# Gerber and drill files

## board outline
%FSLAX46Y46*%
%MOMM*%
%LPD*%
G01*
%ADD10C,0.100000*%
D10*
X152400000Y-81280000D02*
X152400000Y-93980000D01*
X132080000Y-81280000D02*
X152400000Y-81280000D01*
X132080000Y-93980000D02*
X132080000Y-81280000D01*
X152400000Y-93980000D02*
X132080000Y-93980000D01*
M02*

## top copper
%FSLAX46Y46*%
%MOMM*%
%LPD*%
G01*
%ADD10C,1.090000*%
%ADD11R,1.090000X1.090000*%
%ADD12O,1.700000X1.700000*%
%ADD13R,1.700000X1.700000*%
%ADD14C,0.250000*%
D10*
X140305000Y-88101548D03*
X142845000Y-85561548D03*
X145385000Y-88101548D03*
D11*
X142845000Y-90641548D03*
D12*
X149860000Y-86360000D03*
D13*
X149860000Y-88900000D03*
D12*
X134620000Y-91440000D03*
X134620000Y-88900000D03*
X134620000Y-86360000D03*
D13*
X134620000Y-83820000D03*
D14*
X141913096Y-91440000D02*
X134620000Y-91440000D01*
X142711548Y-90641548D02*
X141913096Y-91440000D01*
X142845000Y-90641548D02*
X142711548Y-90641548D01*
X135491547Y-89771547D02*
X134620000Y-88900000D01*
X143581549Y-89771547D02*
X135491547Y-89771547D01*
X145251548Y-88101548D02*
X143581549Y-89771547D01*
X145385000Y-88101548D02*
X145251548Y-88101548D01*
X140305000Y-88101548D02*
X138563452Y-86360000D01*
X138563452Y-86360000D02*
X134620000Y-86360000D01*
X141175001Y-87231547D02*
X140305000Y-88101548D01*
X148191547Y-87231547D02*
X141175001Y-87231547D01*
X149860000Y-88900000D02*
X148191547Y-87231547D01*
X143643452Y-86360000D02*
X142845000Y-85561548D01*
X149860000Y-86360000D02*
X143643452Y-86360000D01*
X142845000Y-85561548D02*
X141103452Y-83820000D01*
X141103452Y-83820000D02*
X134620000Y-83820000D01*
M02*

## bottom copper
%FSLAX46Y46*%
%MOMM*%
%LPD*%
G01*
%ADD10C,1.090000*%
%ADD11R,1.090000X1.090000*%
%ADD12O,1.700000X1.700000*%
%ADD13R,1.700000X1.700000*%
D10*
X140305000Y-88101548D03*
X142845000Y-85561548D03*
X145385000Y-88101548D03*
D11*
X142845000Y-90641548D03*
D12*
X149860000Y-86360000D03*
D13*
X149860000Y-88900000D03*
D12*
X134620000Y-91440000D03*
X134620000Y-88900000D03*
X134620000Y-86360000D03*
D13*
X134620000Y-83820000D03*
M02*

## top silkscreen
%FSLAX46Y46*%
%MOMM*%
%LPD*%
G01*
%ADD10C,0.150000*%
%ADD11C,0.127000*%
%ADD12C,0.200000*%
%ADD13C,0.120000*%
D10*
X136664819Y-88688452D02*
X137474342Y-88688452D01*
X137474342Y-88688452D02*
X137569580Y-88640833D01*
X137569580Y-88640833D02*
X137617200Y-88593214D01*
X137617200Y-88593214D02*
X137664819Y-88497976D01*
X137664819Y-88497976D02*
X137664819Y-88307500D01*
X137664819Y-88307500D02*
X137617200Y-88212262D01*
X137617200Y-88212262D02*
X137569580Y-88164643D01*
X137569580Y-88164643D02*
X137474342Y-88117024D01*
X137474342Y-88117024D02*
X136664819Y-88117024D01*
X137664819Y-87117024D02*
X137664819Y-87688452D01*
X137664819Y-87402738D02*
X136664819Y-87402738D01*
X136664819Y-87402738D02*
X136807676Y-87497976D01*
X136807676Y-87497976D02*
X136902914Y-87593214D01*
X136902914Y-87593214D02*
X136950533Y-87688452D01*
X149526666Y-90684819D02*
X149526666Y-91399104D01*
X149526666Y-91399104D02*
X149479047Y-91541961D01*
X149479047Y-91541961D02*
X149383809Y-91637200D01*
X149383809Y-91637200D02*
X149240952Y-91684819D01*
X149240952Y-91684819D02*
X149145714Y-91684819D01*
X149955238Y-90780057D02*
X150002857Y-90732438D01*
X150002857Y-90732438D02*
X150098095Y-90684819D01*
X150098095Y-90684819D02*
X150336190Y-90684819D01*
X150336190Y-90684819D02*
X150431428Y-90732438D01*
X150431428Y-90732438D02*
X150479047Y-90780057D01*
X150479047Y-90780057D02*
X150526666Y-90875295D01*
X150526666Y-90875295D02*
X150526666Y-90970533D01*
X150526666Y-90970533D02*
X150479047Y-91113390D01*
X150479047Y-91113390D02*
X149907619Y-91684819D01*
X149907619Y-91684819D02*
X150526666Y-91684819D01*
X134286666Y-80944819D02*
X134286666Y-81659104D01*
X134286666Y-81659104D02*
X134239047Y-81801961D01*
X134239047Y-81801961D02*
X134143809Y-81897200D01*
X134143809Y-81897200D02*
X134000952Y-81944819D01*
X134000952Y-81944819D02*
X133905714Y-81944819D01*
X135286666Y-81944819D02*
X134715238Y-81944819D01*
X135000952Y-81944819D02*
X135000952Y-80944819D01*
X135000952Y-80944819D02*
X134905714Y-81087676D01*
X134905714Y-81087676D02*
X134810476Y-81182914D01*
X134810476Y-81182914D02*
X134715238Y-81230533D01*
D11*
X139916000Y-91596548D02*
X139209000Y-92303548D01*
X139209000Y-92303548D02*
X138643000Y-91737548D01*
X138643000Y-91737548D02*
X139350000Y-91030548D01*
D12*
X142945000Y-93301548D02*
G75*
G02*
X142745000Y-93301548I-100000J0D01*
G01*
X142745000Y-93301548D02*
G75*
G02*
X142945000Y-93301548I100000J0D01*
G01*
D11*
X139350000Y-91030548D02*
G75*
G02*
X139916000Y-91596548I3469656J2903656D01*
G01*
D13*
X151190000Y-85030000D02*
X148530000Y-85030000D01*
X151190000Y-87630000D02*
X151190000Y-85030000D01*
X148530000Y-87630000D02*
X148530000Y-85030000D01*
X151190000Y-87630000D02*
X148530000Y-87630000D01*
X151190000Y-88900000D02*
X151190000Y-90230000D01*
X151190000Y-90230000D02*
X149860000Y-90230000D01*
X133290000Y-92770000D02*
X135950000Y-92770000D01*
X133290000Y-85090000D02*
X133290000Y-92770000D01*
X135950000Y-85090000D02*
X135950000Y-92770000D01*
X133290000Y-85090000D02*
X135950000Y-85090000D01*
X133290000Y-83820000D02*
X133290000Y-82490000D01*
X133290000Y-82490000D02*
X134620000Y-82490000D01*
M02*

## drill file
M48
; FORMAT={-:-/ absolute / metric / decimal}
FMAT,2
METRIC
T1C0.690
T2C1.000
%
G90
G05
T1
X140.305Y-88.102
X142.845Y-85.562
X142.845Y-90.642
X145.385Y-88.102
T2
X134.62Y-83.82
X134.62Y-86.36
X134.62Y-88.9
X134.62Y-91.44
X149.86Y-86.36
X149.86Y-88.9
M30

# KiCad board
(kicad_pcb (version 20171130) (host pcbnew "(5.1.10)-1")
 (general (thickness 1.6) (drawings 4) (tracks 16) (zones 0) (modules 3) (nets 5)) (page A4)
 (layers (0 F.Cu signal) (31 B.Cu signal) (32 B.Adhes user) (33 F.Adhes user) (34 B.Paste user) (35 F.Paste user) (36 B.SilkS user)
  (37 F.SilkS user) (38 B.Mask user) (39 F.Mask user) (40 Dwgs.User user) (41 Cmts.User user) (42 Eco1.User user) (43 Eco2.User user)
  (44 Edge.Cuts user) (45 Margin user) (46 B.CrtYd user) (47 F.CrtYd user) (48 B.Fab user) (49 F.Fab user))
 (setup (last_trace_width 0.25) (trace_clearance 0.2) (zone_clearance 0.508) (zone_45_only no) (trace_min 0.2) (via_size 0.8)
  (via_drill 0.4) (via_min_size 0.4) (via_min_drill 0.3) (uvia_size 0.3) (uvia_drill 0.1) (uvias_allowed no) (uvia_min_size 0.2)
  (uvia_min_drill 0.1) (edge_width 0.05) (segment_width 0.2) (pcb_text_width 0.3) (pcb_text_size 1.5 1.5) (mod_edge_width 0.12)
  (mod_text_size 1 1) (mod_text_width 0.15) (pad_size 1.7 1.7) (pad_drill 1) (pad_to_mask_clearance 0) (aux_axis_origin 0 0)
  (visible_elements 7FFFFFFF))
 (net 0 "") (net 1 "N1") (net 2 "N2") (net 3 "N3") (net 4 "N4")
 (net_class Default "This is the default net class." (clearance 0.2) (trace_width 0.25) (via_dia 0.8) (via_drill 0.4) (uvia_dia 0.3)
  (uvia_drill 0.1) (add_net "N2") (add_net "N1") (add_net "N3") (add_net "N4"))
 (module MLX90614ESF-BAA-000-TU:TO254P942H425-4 (layer F.Cu) (at 142.845 88.101548 90)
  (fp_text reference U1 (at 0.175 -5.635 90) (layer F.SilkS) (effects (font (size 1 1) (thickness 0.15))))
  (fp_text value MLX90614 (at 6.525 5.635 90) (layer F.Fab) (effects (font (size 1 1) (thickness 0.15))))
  (fp_line (start -3.495 -2.929) (end -4.202 -3.636) (layer F.SilkS) (width 0.127))
  (fp_line (start -4.202 -3.636) (end -3.636 -4.202) (layer F.SilkS) (width 0.127))
  (fp_line (start -3.636 -4.202) (end -2.929 -3.495) (layer F.SilkS) (width 0.127))
  (fp_circle (center -5.2 0) (end -5.1 0) (layer F.SilkS) (width 0.2))
  (fp_arc (start -0.025344 -0.025344) (end -3.495 -2.929) (angle -349.85) (layer F.SilkS) (width 0.127))
  (pad 4 thru_hole circle (at 0 -2.54 90) (size 1.09 1.09) (drill 0.69) (layers *.Cu *.Mask) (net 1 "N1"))
  (pad 3 thru_hole circle (at 2.54 0 90) (size 1.09 1.09) (drill 0.69) (layers *.Cu *.Mask) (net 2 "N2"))
  (pad 2 thru_hole circle (at 0 2.54 90) (size 1.09 1.09) (drill 0.69) (layers *.Cu *.Mask) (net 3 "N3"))
  (pad 1 thru_hole rect (at -2.54 0 90) (size 1.09 1.09) (drill 0.69) (layers *.Cu *.Mask) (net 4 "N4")))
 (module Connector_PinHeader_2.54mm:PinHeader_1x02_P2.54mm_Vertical (layer F.Cu) (at 149.86 88.9 180)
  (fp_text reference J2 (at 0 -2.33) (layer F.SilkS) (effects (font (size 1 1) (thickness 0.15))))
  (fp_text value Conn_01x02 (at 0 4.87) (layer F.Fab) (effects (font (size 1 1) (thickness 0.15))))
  (fp_line (start -1.33 3.87) (end 1.33 3.87) (layer F.SilkS) (width 0.12))
  (fp_line (start -1.33 1.27) (end -1.33 3.87) (layer F.SilkS) (width 0.12))
  (fp_line (start 1.33 1.27) (end 1.33 3.87) (layer F.SilkS) (width 0.12))
  (fp_line (start -1.33 1.27) (end 1.33 1.27) (layer F.SilkS) (width 0.12))
  (fp_line (start -1.33 0) (end -1.33 -1.33) (layer F.SilkS) (width 0.12))
  (fp_line (start -1.33 -1.33) (end 0 -1.33) (layer F.SilkS) (width 0.12))
  (pad 2 thru_hole oval (at 0 2.54 180) (size 1.7 1.7) (drill 1) (layers *.Cu *.Mask) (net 2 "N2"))
  (pad 1 thru_hole rect (at 0 0 180) (size 1.7 1.7) (drill 1) (layers *.Cu *.Mask) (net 1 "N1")))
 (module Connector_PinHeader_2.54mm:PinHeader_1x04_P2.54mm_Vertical (layer F.Cu) (at 134.62 83.82)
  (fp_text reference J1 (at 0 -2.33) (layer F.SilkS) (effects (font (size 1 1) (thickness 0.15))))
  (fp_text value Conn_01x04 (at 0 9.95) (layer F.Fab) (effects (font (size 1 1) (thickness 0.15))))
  (fp_line (start -1.33 8.95) (end 1.33 8.95) (layer F.SilkS) (width 0.12))
  (fp_line (start -1.33 1.27) (end -1.33 8.95) (layer F.SilkS) (width 0.12))
  (fp_line (start 1.33 1.27) (end 1.33 8.95) (layer F.SilkS) (width 0.12))
  (fp_line (start -1.33 1.27) (end 1.33 1.27) (layer F.SilkS) (width 0.12))
  (fp_line (start -1.33 0) (end -1.33 -1.33) (layer F.SilkS) (width 0.12))
  (fp_line (start -1.33 -1.33) (end 0 -1.33) (layer F.SilkS) (width 0.12))
  (pad 4 thru_hole oval (at 0 7.62) (size 1.7 1.7) (drill 1) (layers *.Cu *.Mask) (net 4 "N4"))
  (pad 3 thru_hole oval (at 0 5.08) (size 1.7 1.7) (drill 1) (layers *.Cu *.Mask) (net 3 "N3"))
  (pad 2 thru_hole oval (at 0 2.54) (size 1.7 1.7) (drill 1) (layers *.Cu *.Mask) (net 1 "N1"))
  (pad 1 thru_hole rect (at 0 0) (size 1.7 1.7) (drill 1) (layers *.Cu *.Mask) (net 2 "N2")))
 (gr_line (start 152.4 81.28) (end 152.4 93.98) (layer Edge.Cuts) (width 0.1))
 (gr_line (start 132.08 81.28) (end 152.4 81.28) (layer Edge.Cuts) (width 0.1))
 (gr_line (start 132.08 93.98) (end 132.08 81.28) (layer Edge.Cuts) (width 0.1))
 (gr_line (start 152.4 93.98) (end 132.08 93.98) (layer Edge.Cuts) (width 0.1))
 (segment (start 141.913096 91.44) (end 134.62 91.44) (width 0.25) (layer F.Cu) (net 4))
 (segment (start 142.711548 90.641548) (end 141.913096 91.44) (width 0.25) (layer F.Cu) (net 4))
 (segment (start 142.845 90.641548) (end 142.711548 90.641548) (width 0.25) (layer F.Cu) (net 4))
 (segment (start 135.491547 89.771547) (end 134.62 88.9) (width 0.25) (layer F.Cu) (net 3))
 (segment (start 143.581549 89.771547) (end 135.491547 89.771547) (width 0.25) (layer F.Cu) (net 3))
 (segment (start 145.251548 88.101548) (end 143.581549 89.771547) (width 0.25) (layer F.Cu) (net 3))
 (segment (start 145.385 88.101548) (end 145.251548 88.101548) (width 0.25) (layer F.Cu) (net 3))
 (segment (start 140.305 88.101548) (end 138.563452 86.36) (width 0.25) (layer F.Cu) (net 1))
 (segment (start 138.563452 86.36) (end 134.62 86.36) (width 0.25) (layer F.Cu) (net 1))
 (segment (start 141.175001 87.231547) (end 140.305 88.101548) (width 0.25) (layer F.Cu) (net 1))
 (segment (start 148.191547 87.231547) (end 141.175001 87.231547) (width 0.25) (layer F.Cu) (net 1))
 (segment (start 149.86 88.9) (end 148.191547 87.231547) (width 0.25) (layer F.Cu) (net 1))
 (segment (start 143.643452 86.36) (end 142.845 85.561548) (width 0.25) (layer F.Cu) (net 2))
 (segment (start 149.86 86.36) (end 143.643452 86.36) (width 0.25) (layer F.Cu) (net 2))
 (segment (start 142.845 85.561548) (end 141.103452 83.82) (width 0.25) (layer F.Cu) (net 2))
 (segment (start 141.103452 83.82) (end 134.62 83.82) (width 0.25) (layer F.Cu) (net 2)))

